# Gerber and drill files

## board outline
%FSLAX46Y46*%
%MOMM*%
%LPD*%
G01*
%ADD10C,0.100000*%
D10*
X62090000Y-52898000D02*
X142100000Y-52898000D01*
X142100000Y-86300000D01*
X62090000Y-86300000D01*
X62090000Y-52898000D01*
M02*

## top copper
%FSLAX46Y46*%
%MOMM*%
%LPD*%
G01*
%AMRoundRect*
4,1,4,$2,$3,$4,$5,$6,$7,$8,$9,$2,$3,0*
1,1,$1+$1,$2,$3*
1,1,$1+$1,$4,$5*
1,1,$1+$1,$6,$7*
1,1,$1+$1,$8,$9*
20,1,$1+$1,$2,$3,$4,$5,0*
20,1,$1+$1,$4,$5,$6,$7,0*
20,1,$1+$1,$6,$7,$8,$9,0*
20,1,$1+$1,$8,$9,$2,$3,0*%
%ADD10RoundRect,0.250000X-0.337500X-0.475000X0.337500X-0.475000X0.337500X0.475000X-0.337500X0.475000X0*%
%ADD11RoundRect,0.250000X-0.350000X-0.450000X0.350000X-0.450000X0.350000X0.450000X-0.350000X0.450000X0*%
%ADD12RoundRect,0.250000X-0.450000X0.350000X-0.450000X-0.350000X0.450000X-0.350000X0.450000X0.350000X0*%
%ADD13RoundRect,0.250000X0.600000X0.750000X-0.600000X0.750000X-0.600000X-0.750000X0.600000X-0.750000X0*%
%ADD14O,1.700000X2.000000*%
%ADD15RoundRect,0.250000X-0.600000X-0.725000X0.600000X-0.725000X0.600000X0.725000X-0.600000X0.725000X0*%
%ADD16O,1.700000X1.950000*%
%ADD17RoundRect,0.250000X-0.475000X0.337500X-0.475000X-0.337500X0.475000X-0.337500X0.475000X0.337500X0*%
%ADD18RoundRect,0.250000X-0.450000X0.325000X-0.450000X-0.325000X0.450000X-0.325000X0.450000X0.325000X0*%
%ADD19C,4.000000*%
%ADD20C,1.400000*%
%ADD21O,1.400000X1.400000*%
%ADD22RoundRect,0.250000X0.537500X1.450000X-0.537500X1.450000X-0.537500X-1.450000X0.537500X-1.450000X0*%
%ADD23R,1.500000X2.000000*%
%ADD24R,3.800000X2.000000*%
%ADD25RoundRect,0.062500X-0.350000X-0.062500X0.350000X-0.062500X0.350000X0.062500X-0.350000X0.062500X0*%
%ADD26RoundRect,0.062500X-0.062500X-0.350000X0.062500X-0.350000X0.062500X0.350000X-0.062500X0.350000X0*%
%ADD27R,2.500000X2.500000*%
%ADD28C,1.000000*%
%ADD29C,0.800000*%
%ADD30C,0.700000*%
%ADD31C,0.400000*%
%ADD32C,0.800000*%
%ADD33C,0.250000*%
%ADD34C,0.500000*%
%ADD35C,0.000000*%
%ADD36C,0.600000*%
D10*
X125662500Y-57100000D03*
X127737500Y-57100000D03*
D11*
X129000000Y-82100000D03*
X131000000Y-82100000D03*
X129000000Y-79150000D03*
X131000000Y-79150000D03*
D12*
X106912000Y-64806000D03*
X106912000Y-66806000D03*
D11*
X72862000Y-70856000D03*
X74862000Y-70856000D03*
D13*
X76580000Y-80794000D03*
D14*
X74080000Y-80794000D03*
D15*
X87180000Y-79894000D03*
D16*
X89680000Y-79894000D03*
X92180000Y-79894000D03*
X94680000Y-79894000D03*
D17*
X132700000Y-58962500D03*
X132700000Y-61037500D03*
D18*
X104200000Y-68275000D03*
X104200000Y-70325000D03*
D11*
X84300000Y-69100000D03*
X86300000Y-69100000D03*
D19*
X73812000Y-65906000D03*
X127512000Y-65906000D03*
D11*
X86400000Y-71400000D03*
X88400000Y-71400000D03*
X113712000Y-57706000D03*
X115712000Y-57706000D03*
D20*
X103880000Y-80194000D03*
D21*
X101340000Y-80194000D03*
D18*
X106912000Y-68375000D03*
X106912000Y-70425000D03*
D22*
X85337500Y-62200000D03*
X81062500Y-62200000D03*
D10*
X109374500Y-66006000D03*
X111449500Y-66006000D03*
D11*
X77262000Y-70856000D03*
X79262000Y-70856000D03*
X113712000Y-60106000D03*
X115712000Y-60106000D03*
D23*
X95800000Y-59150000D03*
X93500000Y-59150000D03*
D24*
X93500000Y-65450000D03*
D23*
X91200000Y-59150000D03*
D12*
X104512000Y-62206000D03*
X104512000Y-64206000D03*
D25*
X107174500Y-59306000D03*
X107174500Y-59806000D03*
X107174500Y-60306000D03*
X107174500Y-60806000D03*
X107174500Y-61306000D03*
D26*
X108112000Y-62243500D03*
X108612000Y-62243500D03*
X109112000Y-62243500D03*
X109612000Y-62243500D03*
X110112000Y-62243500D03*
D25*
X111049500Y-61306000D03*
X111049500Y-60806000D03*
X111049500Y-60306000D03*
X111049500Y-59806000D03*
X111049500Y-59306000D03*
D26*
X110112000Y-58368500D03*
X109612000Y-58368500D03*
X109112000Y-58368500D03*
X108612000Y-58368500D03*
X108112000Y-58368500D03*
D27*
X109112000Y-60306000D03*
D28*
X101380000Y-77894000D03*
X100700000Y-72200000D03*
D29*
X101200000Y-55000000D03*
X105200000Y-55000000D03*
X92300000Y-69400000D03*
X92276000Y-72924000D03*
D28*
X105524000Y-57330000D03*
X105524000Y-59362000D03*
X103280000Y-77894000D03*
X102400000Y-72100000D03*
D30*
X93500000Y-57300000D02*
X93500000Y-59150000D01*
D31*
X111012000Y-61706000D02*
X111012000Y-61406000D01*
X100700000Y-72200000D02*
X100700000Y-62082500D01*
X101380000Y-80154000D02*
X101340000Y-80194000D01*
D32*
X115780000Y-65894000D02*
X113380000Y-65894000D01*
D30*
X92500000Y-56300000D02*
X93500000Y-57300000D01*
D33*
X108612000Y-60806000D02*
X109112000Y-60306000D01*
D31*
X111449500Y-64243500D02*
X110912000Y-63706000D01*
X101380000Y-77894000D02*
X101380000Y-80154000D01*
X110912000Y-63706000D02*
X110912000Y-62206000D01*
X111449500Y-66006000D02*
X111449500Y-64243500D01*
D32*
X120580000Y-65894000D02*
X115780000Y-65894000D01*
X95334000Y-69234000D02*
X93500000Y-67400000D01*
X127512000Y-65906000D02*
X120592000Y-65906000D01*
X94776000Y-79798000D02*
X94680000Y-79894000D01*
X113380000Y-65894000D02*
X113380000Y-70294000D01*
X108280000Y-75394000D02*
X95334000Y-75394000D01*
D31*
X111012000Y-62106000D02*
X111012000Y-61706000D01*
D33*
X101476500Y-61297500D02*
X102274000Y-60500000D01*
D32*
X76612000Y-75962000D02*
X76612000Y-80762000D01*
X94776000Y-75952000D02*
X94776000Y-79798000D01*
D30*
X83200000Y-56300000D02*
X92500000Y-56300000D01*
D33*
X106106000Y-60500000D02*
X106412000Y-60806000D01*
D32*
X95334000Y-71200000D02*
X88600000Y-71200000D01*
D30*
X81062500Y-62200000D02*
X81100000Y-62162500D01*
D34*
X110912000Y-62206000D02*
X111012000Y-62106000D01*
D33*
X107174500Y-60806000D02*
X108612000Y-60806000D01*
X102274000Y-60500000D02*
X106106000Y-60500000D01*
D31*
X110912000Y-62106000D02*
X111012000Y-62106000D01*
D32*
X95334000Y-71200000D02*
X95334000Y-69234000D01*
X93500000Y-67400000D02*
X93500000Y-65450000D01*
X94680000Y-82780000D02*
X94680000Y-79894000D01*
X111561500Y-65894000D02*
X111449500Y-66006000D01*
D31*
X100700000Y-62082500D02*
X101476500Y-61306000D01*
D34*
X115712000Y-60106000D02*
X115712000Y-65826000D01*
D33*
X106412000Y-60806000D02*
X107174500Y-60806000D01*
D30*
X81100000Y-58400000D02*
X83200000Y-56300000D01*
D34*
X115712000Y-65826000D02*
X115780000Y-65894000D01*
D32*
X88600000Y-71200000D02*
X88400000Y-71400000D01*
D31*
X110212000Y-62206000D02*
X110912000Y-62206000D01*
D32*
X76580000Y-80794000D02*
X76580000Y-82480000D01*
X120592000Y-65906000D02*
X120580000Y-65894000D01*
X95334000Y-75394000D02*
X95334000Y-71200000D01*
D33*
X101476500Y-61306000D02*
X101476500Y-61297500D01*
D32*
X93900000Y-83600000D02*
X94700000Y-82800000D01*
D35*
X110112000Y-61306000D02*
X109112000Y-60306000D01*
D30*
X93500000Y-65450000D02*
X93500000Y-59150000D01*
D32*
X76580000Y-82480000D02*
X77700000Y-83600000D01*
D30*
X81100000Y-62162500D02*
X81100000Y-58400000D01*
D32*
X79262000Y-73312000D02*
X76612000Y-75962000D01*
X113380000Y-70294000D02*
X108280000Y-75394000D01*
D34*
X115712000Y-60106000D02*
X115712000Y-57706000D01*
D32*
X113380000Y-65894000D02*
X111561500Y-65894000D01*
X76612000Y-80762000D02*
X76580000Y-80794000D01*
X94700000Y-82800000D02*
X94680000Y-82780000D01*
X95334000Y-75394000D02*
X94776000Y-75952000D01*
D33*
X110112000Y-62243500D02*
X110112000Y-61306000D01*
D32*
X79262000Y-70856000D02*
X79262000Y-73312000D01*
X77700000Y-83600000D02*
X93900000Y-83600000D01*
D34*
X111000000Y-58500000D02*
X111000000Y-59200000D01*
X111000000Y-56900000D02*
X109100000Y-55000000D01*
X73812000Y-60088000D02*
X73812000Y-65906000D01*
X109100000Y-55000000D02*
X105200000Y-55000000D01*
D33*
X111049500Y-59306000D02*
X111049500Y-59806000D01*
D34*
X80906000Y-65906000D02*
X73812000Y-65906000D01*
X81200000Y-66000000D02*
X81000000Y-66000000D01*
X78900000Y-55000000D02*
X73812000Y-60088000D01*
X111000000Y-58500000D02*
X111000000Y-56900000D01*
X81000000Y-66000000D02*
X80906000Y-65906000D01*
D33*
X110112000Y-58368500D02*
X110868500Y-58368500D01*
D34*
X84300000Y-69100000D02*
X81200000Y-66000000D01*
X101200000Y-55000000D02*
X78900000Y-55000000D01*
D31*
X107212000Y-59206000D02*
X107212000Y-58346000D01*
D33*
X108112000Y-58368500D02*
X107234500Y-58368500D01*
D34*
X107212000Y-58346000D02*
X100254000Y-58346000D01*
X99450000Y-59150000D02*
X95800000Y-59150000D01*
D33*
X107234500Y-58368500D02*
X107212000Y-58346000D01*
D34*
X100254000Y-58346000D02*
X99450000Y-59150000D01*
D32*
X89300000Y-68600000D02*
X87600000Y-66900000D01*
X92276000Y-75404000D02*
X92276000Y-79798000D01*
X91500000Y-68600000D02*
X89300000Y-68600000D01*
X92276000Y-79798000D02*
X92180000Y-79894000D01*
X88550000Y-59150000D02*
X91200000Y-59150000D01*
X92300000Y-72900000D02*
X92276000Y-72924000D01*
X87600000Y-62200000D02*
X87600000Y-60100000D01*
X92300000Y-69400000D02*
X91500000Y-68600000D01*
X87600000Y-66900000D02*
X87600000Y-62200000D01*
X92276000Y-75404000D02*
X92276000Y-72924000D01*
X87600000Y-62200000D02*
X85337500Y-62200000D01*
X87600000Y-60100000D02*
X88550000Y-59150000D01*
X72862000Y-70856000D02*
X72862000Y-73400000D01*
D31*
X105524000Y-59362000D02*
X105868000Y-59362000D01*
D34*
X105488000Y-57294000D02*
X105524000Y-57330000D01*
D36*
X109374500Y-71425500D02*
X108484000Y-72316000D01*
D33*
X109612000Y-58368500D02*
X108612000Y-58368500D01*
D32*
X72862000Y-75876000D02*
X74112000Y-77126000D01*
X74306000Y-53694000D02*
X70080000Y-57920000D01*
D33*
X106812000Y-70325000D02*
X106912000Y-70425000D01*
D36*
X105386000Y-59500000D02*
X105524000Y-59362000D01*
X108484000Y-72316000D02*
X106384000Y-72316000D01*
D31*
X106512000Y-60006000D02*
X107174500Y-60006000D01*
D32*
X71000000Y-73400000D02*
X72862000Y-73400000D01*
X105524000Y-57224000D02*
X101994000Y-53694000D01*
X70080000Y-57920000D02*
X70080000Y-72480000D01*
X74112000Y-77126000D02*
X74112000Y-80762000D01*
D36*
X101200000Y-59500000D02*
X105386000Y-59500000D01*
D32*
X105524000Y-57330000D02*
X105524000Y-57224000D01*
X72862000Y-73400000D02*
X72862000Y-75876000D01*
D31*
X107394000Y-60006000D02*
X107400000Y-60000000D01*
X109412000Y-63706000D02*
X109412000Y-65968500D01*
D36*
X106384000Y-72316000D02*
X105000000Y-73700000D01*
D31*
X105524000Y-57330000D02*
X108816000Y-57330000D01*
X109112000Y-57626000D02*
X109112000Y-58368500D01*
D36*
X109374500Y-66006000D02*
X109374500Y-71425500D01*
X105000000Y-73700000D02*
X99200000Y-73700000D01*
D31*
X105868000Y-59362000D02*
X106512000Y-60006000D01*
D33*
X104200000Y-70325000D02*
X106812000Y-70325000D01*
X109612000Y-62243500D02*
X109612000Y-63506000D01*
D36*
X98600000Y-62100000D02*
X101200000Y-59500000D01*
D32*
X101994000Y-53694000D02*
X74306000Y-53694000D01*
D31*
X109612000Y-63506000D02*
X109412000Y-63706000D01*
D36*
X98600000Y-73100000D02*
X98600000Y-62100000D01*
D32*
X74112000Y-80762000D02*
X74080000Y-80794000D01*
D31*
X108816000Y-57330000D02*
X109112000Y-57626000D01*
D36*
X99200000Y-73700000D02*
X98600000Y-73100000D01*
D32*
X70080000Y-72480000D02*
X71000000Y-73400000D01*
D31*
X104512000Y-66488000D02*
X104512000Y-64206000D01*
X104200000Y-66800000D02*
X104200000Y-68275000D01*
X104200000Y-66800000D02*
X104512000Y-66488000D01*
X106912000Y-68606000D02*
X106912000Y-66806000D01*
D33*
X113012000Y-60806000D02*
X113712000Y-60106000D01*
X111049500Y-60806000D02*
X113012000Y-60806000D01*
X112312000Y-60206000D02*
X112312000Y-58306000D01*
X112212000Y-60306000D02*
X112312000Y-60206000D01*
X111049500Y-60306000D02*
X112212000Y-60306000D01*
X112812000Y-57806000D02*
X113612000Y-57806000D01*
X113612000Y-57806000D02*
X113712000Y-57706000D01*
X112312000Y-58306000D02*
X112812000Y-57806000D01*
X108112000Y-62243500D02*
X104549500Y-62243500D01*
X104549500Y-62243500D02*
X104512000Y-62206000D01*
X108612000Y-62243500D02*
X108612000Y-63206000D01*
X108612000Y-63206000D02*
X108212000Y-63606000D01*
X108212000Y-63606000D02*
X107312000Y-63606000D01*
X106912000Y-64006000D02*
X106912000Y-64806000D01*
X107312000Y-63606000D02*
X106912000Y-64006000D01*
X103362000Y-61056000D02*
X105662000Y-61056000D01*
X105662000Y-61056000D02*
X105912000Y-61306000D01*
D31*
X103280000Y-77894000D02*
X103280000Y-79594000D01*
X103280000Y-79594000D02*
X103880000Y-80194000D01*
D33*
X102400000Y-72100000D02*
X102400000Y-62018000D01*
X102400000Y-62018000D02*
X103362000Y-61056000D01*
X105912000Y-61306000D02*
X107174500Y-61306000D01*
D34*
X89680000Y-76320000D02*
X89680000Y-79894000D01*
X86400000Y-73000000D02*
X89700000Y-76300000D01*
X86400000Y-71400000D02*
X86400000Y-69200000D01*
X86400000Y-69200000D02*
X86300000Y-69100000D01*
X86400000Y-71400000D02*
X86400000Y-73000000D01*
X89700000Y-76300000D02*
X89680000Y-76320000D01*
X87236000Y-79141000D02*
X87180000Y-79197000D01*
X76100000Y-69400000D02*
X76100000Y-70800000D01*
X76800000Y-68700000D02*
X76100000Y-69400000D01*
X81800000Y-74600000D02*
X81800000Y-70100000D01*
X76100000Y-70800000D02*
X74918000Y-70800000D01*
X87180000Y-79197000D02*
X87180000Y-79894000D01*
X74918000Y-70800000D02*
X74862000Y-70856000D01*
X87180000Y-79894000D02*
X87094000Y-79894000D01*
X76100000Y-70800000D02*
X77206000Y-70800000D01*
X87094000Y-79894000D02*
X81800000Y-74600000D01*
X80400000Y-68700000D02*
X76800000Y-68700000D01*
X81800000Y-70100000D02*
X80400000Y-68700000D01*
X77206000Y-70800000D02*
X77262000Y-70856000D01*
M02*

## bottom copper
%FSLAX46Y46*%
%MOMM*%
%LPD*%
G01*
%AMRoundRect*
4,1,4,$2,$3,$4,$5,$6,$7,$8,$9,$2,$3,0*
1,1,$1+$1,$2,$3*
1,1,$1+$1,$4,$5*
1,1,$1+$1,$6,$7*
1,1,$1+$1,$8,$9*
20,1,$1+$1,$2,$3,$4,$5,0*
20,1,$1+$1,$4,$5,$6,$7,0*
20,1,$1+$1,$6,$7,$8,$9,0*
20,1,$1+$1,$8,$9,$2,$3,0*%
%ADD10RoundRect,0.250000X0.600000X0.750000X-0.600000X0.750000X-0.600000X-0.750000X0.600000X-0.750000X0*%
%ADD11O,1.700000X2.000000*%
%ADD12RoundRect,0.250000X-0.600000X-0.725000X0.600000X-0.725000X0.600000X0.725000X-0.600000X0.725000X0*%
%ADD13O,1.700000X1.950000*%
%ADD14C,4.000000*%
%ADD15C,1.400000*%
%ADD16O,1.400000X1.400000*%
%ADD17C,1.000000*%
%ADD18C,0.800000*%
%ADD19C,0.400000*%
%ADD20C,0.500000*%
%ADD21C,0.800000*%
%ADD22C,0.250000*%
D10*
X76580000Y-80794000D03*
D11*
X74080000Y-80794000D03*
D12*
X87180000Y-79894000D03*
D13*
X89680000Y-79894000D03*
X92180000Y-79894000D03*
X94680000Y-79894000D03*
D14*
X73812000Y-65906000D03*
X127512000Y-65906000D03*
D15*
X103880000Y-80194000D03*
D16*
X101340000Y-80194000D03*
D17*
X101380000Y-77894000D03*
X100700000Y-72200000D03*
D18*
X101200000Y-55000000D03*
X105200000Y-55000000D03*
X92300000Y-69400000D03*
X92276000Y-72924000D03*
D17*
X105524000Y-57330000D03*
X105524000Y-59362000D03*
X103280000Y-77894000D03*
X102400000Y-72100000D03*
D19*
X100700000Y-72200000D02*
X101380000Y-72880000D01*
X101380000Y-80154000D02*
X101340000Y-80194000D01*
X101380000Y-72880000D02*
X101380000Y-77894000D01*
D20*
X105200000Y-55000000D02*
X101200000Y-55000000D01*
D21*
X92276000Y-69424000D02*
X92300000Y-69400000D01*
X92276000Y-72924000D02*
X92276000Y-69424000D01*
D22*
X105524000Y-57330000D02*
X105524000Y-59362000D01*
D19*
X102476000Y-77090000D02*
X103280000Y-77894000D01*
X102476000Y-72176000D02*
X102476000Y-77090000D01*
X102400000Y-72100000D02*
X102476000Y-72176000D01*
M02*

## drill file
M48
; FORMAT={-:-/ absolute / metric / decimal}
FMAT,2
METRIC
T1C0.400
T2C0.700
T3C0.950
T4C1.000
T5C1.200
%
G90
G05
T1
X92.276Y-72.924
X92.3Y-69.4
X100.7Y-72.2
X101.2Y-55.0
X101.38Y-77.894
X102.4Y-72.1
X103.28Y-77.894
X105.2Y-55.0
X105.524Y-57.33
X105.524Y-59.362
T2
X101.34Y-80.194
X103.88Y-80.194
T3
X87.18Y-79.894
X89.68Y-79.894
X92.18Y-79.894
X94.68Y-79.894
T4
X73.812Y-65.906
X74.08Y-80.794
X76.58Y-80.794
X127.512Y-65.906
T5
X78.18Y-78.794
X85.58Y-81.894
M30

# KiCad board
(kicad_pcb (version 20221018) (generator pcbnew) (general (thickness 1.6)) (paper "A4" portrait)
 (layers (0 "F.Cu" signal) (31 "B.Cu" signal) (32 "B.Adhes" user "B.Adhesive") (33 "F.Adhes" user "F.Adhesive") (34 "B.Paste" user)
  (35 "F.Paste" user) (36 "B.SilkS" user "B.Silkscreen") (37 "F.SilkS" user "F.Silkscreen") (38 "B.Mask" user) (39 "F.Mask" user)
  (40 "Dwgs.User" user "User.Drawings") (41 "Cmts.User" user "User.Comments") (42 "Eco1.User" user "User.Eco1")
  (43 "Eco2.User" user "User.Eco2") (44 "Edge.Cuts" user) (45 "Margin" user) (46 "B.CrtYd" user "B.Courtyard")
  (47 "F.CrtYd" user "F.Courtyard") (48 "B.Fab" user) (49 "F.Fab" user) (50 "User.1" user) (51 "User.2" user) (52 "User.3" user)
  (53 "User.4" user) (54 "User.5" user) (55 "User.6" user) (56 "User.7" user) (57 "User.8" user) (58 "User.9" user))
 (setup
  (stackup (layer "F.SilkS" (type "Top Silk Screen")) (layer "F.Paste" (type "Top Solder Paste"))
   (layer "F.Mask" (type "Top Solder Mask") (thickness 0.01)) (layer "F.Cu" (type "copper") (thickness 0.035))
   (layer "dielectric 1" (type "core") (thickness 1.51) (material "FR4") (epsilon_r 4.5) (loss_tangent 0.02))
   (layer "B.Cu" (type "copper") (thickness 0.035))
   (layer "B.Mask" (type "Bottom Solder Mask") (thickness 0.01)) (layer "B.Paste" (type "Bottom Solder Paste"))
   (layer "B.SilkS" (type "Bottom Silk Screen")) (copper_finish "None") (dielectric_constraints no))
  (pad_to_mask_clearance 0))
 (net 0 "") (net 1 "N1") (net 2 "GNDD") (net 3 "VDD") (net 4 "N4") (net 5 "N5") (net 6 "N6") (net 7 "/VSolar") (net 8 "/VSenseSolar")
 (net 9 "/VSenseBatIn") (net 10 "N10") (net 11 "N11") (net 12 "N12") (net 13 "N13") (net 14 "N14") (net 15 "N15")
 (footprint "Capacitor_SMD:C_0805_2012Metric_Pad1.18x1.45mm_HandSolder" (layer "F.Cu") (at 126.7 57.1)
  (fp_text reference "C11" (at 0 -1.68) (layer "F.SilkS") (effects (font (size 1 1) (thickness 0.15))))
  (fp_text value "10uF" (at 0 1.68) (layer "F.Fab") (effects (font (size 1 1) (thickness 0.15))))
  (pad "1" smd roundrect (at -1.0375 0) (size 1.175 1.45) (layers "F.Cu" "F.Paste" "F.Mask") (roundrect_rratio 0.212766) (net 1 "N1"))
  (pad "2" smd roundrect (at 1.0375 0) (size 1.175 1.45) (layers "F.Cu" "F.Paste" "F.Mask") (roundrect_rratio 0.212766) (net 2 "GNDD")))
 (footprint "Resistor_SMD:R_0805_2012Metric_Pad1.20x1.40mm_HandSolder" (layer "F.Cu") (at 130 82.1)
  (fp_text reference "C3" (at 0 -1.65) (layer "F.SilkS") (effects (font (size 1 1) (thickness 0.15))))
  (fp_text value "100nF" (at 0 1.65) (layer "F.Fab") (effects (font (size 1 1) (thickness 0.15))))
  (pad "1" smd roundrect (at -1 0) (size 1.2 1.4) (layers "F.Cu" "F.Paste" "F.Mask") (roundrect_rratio 0.208333) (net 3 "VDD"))
  (pad "2" smd roundrect (at 1 0) (size 1.2 1.4) (layers "F.Cu" "F.Paste" "F.Mask") (roundrect_rratio 0.208333) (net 2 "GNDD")))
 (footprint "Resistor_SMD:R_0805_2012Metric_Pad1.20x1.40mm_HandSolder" (layer "F.Cu") (at 130 79.15)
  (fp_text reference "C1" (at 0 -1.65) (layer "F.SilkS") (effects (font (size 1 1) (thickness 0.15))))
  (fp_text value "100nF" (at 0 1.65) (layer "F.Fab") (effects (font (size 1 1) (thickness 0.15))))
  (pad "1" smd roundrect (at -1 0) (size 1.2 1.4) (layers "F.Cu" "F.Paste" "F.Mask") (roundrect_rratio 0.208333) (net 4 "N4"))
  (pad "2" smd roundrect (at 1 0) (size 1.2 1.4) (layers "F.Cu" "F.Paste" "F.Mask") (roundrect_rratio 0.208333) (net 2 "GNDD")))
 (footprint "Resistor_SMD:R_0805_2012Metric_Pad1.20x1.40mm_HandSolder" (layer "F.Cu") (at 106.912 65.806 -90)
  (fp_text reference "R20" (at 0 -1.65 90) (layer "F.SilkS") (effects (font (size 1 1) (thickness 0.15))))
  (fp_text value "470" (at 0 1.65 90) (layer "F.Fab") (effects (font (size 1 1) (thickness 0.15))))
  (pad "1" smd roundrect (at -1 0 270) (size 1.2 1.4) (layers "F.Cu" "F.Paste" "F.Mask") (roundrect_rratio 0.208333) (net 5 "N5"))
  (pad "2" smd roundrect (at 1 0 270) (size 1.2 1.4) (layers "F.Cu" "F.Paste" "F.Mask") (roundrect_rratio 0.208333) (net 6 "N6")))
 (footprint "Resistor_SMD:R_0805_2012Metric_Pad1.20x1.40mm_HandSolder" (layer "F.Cu") (at 73.862 70.856)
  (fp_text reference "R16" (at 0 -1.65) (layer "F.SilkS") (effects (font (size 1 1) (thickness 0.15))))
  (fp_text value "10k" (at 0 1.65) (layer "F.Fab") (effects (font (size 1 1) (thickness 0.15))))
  (pad "1" smd roundrect (at -1 0) (size 1.2 1.4) (layers "F.Cu" "F.Paste" "F.Mask") (roundrect_rratio 0.208333) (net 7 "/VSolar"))
  (pad "2" smd roundrect (at 1 0) (size 1.2 1.4) (layers "F.Cu" "F.Paste" "F.Mask") (roundrect_rratio 0.208333) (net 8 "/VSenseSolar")))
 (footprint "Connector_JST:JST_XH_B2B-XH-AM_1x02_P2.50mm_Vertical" (layer "F.Cu") (at 76.58 80.794 180)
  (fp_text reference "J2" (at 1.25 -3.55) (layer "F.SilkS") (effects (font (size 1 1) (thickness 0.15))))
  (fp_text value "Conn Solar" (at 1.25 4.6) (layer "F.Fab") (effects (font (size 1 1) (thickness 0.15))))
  (pad "" np_thru_hole circle (at -1.6 2 180) (size 1.2 1.2) (drill 1.2) (layers "*.Cu" "*.Mask"))
  (pad "1" thru_hole roundrect (at 0 0 180) (size 1.7 2) (drill 1) (layers "*.Cu" "*.Mask") (roundrect_rratio 0.147059) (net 2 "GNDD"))
  (pad "2" thru_hole oval (at 2.5 0 180) (size 1.7 2) (drill 1) (layers "*.Cu" "*.Mask") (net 7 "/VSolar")))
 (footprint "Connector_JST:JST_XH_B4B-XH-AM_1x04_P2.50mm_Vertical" (layer "F.Cu") (at 87.18 79.894)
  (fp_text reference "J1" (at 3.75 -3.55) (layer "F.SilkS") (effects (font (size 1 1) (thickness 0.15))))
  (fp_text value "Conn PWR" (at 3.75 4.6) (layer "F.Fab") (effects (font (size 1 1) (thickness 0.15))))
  (pad "" np_thru_hole circle (at -1.6 2) (size 1.2 1.2) (drill 1.2) (layers "*.Cu" "*.Mask"))
  (pad "1" thru_hole roundrect (at 0 0) (size 1.7 1.95) (drill 0.95) (layers "*.Cu" "*.Mask") (roundrect_rratio 0.147059)
   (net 8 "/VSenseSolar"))
  (pad "2" thru_hole oval (at 2.5 0) (size 1.7 1.95) (drill 0.95) (layers "*.Cu" "*.Mask") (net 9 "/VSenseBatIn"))
  (pad "3" thru_hole oval (at 5 0) (size 1.7 1.95) (drill 0.95) (layers "*.Cu" "*.Mask") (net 3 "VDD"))
  (pad "4" thru_hole oval (at 7.5 0) (size 1.7 1.95) (drill 0.95) (layers "*.Cu" "*.Mask") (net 2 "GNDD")))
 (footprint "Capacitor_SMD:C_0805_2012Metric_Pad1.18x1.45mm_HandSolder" (layer "F.Cu") (at 132.7 60 -90)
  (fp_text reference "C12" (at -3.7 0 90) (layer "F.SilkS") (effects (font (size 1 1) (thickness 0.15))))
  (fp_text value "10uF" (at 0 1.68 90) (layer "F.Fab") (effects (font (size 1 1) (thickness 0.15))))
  (pad "1" smd roundrect (at -1.0375 0 270) (size 1.175 1.45) (layers "F.Cu" "F.Paste" "F.Mask") (roundrect_rratio 0.212766) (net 4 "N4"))
  (pad "2" smd roundrect (at 1.0375 0 270) (size 1.175 1.45) (layers "F.Cu" "F.Paste" "F.Mask") (roundrect_rratio 0.212766) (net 2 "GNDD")))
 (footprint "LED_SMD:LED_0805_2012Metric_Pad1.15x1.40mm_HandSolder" (layer "F.Cu") (at 104.2 69.3 -90)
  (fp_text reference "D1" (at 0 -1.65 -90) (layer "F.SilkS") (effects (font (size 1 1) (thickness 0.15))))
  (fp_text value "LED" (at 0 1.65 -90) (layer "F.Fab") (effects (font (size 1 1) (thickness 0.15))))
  (pad "1" smd roundrect (at -1.025 0 270) (size 1.15 1.4) (layers "F.Cu" "F.Paste" "F.Mask") (roundrect_rratio 0.217391) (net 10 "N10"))
  (pad "2" smd roundrect (at 1.025 0 270) (size 1.15 1.4) (layers "F.Cu" "F.Paste" "F.Mask") (roundrect_rratio 0.217391) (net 7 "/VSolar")))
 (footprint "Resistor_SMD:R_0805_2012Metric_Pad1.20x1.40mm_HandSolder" (layer "F.Cu") (at 85.3 69.1)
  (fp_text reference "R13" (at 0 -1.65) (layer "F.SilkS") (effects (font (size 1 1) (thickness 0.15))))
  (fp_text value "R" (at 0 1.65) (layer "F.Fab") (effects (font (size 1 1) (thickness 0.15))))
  (pad "1" smd roundrect (at -1 0) (size 1.2 1.4) (layers "F.Cu" "F.Paste" "F.Mask") (roundrect_rratio 0.208333) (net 1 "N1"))
  (pad "2" smd roundrect (at 1 0) (size 1.2 1.4) (layers "F.Cu" "F.Paste" "F.Mask") (roundrect_rratio 0.208333) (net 9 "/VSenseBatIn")))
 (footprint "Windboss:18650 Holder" (layer "F.Cu") (at 74.512 65.906)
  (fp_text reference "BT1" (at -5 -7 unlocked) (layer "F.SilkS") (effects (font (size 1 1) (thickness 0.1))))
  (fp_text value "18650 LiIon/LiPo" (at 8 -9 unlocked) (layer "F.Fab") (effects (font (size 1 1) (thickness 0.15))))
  (pad "1" thru_hole circle (at -0.7 0) (size 4 4) (drill 1) (layers "*.Cu" "*.Mask") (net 1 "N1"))
  (pad "2" thru_hole circle (at 53 0) (size 4 4) (drill 1) (layers "*.Cu" "*.Mask") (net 2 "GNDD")))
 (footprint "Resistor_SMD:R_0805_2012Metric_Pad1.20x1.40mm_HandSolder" (layer "F.Cu") (at 87.4 71.4)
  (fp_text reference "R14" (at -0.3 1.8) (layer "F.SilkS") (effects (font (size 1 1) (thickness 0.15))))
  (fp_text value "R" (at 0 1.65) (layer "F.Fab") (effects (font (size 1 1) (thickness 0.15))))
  (pad "1" smd roundrect (at -1 0) (size 1.2 1.4) (layers "F.Cu" "F.Paste" "F.Mask") (roundrect_rratio 0.208333) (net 9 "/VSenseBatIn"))
  (pad "2" smd roundrect (at 1 0) (size 1.2 1.4) (layers "F.Cu" "F.Paste" "F.Mask") (roundrect_rratio 0.208333) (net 2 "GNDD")))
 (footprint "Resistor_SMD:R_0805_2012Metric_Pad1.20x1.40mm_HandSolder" (layer "F.Cu") (at 114.712 57.706)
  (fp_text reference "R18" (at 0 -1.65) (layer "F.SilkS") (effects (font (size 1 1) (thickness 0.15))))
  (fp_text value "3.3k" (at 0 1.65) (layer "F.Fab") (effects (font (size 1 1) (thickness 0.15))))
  (pad "1" smd roundrect (at -1 0) (size 1.2 1.4) (layers "F.Cu" "F.Paste" "F.Mask") (roundrect_rratio 0.208333) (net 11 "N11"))
  (pad "2" smd roundrect (at 1 0) (size 1.2 1.4) (layers "F.Cu" "F.Paste" "F.Mask") (roundrect_rratio 0.208333) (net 2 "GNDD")))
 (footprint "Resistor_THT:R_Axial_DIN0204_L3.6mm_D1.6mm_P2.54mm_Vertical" (layer "F.Cu") (at 103.88 80.194 180)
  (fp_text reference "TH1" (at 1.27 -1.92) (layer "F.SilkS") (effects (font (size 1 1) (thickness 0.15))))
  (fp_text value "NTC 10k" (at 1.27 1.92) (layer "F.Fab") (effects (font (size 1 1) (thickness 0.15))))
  (pad "1" thru_hole circle (at 0 0 180) (size 1.4 1.4) (drill 0.7) (layers "*.Cu" "*.Mask") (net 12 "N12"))
  (pad "2" thru_hole oval (at 2.54 0 180) (size 1.4 1.4) (drill 0.7) (layers "*.Cu" "*.Mask") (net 2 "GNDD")))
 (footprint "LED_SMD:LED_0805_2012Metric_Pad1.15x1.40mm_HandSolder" (layer "F.Cu") (at 106.912 69.4 -90)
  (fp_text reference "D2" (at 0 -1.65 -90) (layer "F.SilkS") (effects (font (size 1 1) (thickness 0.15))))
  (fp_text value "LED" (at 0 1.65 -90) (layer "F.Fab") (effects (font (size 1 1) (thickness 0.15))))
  (pad "1" smd roundrect (at -1.025 0 270) (size 1.15 1.4) (layers "F.Cu" "F.Paste" "F.Mask") (roundrect_rratio 0.217391) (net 6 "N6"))
  (pad "2" smd roundrect (at 1.025 0 270) (size 1.15 1.4) (layers "F.Cu" "F.Paste" "F.Mask") (roundrect_rratio 0.217391) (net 7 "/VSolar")))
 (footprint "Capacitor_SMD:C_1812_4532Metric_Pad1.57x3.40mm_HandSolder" (layer "F.Cu") (at 83.2 62.2 180)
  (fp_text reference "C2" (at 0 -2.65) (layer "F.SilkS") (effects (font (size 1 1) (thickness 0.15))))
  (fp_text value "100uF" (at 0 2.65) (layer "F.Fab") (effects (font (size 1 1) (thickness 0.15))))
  (pad "1" smd roundrect (at -2.1375 0 180) (size 1.575 3.4) (layers "F.Cu" "F.Paste" "F.Mask") (roundrect_rratio 0.15873) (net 3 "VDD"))
  (pad "2" smd roundrect (at 2.1375 0 180) (size 1.575 3.4) (layers "F.Cu" "F.Paste" "F.Mask") (roundrect_rratio 0.15873) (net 2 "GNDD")))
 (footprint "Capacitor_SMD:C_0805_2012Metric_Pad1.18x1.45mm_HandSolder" (layer "F.Cu") (at 110.412 66.006)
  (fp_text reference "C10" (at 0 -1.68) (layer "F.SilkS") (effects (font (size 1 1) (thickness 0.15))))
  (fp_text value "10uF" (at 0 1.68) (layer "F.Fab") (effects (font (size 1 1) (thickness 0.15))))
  (pad "1" smd roundrect (at -1.0375 0) (size 1.175 1.45) (layers "F.Cu" "F.Paste" "F.Mask") (roundrect_rratio 0.212766) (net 7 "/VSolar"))
  (pad "2" smd roundrect (at 1.0375 0) (size 1.175 1.45) (layers "F.Cu" "F.Paste" "F.Mask") (roundrect_rratio 0.212766) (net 2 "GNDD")))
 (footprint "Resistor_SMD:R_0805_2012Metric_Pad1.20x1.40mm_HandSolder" (layer "F.Cu") (at 78.262 70.856)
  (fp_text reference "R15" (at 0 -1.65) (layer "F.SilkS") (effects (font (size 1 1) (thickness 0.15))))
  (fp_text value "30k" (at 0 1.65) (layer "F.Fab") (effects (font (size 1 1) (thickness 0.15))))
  (pad "1" smd roundrect (at -1 0) (size 1.2 1.4) (layers "F.Cu" "F.Paste" "F.Mask") (roundrect_rratio 0.208333) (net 8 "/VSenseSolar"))
  (pad "2" smd roundrect (at 1 0) (size 1.2 1.4) (layers "F.Cu" "F.Paste" "F.Mask") (roundrect_rratio 0.208333) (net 2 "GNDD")))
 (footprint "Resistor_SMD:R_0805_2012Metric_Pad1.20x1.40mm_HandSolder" (layer "F.Cu") (at 114.712 60.106)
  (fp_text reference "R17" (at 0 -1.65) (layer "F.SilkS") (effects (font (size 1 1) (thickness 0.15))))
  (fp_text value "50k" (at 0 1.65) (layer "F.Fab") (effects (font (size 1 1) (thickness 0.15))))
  (pad "1" smd roundrect (at -1 0) (size 1.2 1.4) (layers "F.Cu" "F.Paste" "F.Mask") (roundrect_rratio 0.208333) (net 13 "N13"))
  (pad "2" smd roundrect (at 1 0) (size 1.2 1.4) (layers "F.Cu" "F.Paste" "F.Mask") (roundrect_rratio 0.208333) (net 2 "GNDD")))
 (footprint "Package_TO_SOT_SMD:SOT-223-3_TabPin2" (layer "F.Cu") (at 93.5 62.3 -90)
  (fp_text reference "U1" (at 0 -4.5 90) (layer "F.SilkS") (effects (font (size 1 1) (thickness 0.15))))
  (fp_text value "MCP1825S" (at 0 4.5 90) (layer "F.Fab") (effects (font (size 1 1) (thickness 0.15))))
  (pad "1" smd rect (at -3.15 -2.3 270) (size 2 1.5) (layers "F.Cu" "F.Paste" "F.Mask") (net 4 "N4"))
  (pad "2" smd rect (at -3.15 0 270) (size 2 1.5) (layers "F.Cu" "F.Paste" "F.Mask") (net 2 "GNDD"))
  (pad "2" smd rect (at 3.15 0 270) (size 2 3.8) (layers "F.Cu" "F.Paste" "F.Mask") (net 2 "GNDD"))
  (pad "3" smd rect (at -3.15 2.3 270) (size 2 1.5) (layers "F.Cu" "F.Paste" "F.Mask") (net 3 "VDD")))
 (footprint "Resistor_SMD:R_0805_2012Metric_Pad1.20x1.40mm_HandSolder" (layer "F.Cu") (at 104.512 63.206 -90)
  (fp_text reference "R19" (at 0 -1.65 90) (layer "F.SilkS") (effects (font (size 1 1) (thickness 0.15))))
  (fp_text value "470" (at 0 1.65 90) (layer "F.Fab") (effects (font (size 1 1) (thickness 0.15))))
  (pad "1" smd roundrect (at -1 0 270) (size 1.2 1.4) (layers "F.Cu" "F.Paste" "F.Mask") (roundrect_rratio 0.208333) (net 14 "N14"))
  (pad "2" smd roundrect (at 1 0 270) (size 1.2 1.4) (layers "F.Cu" "F.Paste" "F.Mask") (roundrect_rratio 0.208333) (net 10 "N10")))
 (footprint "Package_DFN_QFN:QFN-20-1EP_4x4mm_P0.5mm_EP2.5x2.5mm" (layer "F.Cu") (at 109.112 60.306)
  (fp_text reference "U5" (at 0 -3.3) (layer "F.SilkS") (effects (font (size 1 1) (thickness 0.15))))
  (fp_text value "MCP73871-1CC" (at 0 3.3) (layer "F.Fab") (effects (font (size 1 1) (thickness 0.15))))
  (pad "" smd roundrect (at -0.625 -0.625) (size 1.01 1.01) (layers "F.Paste") (roundrect_rratio 0.247525))
  (pad "" smd roundrect (at -0.625 0.625) (size 1.01 1.01) (layers "F.Paste") (roundrect_rratio 0.247525))
  (pad "" smd roundrect (at 0.625 -0.625) (size 1.01 1.01) (layers "F.Paste") (roundrect_rratio 0.247525))
  (pad "" smd roundrect (at 0.625 0.625) (size 1.01 1.01) (layers "F.Paste") (roundrect_rratio 0.247525))
  (pad "1" smd roundrect (at -1.9375 -1) (size 0.825 0.25) (layers "F.Cu" "F.Paste" "F.Mask") (roundrect_rratio 0.25) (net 4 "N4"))
  (pad "2" smd roundrect (at -1.9375 -0.5) (size 0.825 0.25) (layers "F.Cu" "F.Paste" "F.Mask") (roundrect_rratio 0.25) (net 7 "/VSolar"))
  (pad "3" smd roundrect (at -1.9375 0) (size 0.825 0.25) (layers "F.Cu" "F.Paste" "F.Mask") (roundrect_rratio 0.25) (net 7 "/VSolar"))
  (pad "4" smd roundrect (at -1.9375 0.5) (size 0.825 0.25) (layers "F.Cu" "F.Paste" "F.Mask") (roundrect_rratio 0.25) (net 2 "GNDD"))
  (pad "5" smd roundrect (at -1.9375 1) (size 0.825 0.25) (layers "F.Cu" "F.Paste" "F.Mask") (roundrect_rratio 0.25) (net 12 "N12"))
  (pad "6" smd roundrect (at -1 1.9375) (size 0.25 0.825) (layers "F.Cu" "F.Paste" "F.Mask") (roundrect_rratio 0.25) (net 14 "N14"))
  (pad "7" smd roundrect (at -0.5 1.9375) (size 0.25 0.825) (layers "F.Cu" "F.Paste" "F.Mask") (roundrect_rratio 0.25) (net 5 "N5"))
  (pad "8" smd roundrect (at 0 1.9375) (size 0.25 0.825) (layers "F.Cu" "F.Paste" "F.Mask") (roundrect_rratio 0.25) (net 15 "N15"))
  (pad "9" smd roundrect (at 0.5 1.9375) (size 0.25 0.825) (layers "F.Cu" "F.Paste" "F.Mask") (roundrect_rratio 0.25) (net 7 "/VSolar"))
  (pad "10" smd roundrect (at 1 1.9375) (size 0.25 0.825) (layers "F.Cu" "F.Paste" "F.Mask") (roundrect_rratio 0.25) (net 2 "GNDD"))
  (pad "11" smd roundrect (at 1.9375 1) (size 0.825 0.25) (layers "F.Cu" "F.Paste" "F.Mask") (roundrect_rratio 0.25) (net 2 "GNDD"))
  (pad "12" smd roundrect (at 1.9375 0.5) (size 0.825 0.25) (layers "F.Cu" "F.Paste" "F.Mask") (roundrect_rratio 0.25) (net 13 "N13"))
  (pad "13" smd roundrect (at 1.9375 0) (size 0.825 0.25) (layers "F.Cu" "F.Paste" "F.Mask") (roundrect_rratio 0.25) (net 11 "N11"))
  (pad "14" smd roundrect (at 1.9375 -0.5) (size 0.825 0.25) (layers "F.Cu" "F.Paste" "F.Mask") (roundrect_rratio 0.25) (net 1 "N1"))
  (pad "15" smd roundrect (at 1.9375 -1) (size 0.825 0.25) (layers "F.Cu" "F.Paste" "F.Mask") (roundrect_rratio 0.25) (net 1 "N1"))
  (pad "16" smd roundrect (at 1 -1.9375) (size 0.25 0.825) (layers "F.Cu" "F.Paste" "F.Mask") (roundrect_rratio 0.25) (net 1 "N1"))
  (pad "17" smd roundrect (at 0.5 -1.9375) (size 0.25 0.825) (layers "F.Cu" "F.Paste" "F.Mask") (roundrect_rratio 0.25) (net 7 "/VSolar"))
  (pad "18" smd roundrect (at 0 -1.9375) (size 0.25 0.825) (layers "F.Cu" "F.Paste" "F.Mask") (roundrect_rratio 0.25) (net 7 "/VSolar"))
  (pad "19" smd roundrect (at -0.5 -1.9375) (size 0.25 0.825) (layers "F.Cu" "F.Paste" "F.Mask") (roundrect_rratio 0.25) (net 7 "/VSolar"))
  (pad "20" smd roundrect (at -1 -1.9375) (size 0.25 0.825) (layers "F.Cu" "F.Paste" "F.Mask") (roundrect_rratio 0.25) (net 4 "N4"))
  (pad "21" smd rect (at 0 0) (size 2.5 2.5) (layers "F.Cu" "F.Mask") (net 2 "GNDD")))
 (gr_rect (start 62.09 52.898) (end 142.1 86.3) (stroke (width 0.1) (type default)) (fill none) (layer "Edge.Cuts"))
 (segment (start 93.5 57.3) (end 93.5 59.15) (width 0.7) (layer "F.Cu") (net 2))
 (segment (start 111.012 61.706) (end 111.012 61.406) (width 0.4) (layer "F.Cu") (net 2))
 (segment (start 100.7 72.2) (end 100.7 62.0825) (width 0.4) (layer "F.Cu") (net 2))
 (segment (start 101.38 80.154) (end 101.34 80.194) (width 0.4) (layer "F.Cu") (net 2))
 (segment (start 115.78 65.894) (end 113.38 65.894) (width 0.8) (layer "F.Cu") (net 2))
 (segment (start 92.5 56.3) (end 93.5 57.3) (width 0.7) (layer "F.Cu") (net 2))
 (segment (start 108.612 60.806) (end 109.112 60.306) (width 0.25) (layer "F.Cu") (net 2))
 (segment (start 111.4495 64.2435) (end 110.912 63.706) (width 0.4) (layer "F.Cu") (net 2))
 (segment (start 101.38 77.894) (end 101.38 80.154) (width 0.4) (layer "F.Cu") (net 2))
 (segment (start 110.912 63.706) (end 110.912 62.206) (width 0.4) (layer "F.Cu") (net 2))
 (segment (start 111.4495 66.006) (end 111.4495 64.2435) (width 0.4) (layer "F.Cu") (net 2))
 (segment (start 120.58 65.894) (end 115.78 65.894) (width 0.8) (layer "F.Cu") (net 2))
 (segment (start 95.334 69.234) (end 93.5 67.4) (width 0.8) (layer "F.Cu") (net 2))
 (segment (start 127.512 65.906) (end 120.592 65.906) (width 0.8) (layer "F.Cu") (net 2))
 (segment (start 94.776 79.798) (end 94.68 79.894) (width 0.8) (layer "F.Cu") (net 2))
 (segment (start 113.38 65.894) (end 113.38 70.294) (width 0.8) (layer "F.Cu") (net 2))
 (segment (start 108.28 75.394) (end 95.334 75.394) (width 0.8) (layer "F.Cu") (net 2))
 (segment (start 111.012 62.106) (end 111.012 61.706) (width 0.4) (layer "F.Cu") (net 2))
 (segment (start 101.4765 61.2975) (end 102.274 60.5) (width 0.25) (layer "F.Cu") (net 2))
 (segment (start 76.612 75.962) (end 76.612 80.762) (width 0.8) (layer "F.Cu") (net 2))
 (segment (start 94.776 75.952) (end 94.776 79.798) (width 0.8) (layer "F.Cu") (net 2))
 (segment (start 83.2 56.3) (end 92.5 56.3) (width 0.7) (layer "F.Cu") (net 2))
 (segment (start 106.106 60.5) (end 106.412 60.806) (width 0.25) (layer "F.Cu") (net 2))
 (segment (start 95.334 71.2) (end 88.6 71.2) (width 0.8) (layer "F.Cu") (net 2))
 (segment (start 81.0625 62.2) (end 81.1 62.1625) (width 0.7) (layer "F.Cu") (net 2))
 (segment (start 110.912 62.206) (end 111.012 62.106) (width 0.5) (layer "F.Cu") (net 2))
 (segment (start 107.1745 60.806) (end 108.612 60.806) (width 0.25) (layer "F.Cu") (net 2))
 (segment (start 102.274 60.5) (end 106.106 60.5) (width 0.25) (layer "F.Cu") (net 2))
 (segment (start 110.912 62.106) (end 111.012 62.106) (width 0.4) (layer "F.Cu") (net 2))
 (segment (start 95.334 71.2) (end 95.334 69.234) (width 0.8) (layer "F.Cu") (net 2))
 (segment (start 93.5 67.4) (end 93.5 65.45) (width 0.8) (layer "F.Cu") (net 2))
 (segment (start 94.68 82.78) (end 94.68 79.894) (width 0.8) (layer "F.Cu") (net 2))
 (segment (start 111.5615 65.894) (end 111.4495 66.006) (width 0.8) (layer "F.Cu") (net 2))
 (segment (start 100.7 62.0825) (end 101.4765 61.306) (width 0.4) (layer "F.Cu") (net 2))
 (segment (start 115.712 60.106) (end 115.712 65.826) (width 0.5) (layer "F.Cu") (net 2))
 (segment (start 106.412 60.806) (end 107.1745 60.806) (width 0.25) (layer "F.Cu") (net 2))
 (segment (start 81.1 58.4) (end 83.2 56.3) (width 0.7) (layer "F.Cu") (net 2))
 (segment (start 115.712 65.826) (end 115.78 65.894) (width 0.5) (layer "F.Cu") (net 2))
 (segment (start 88.6 71.2) (end 88.4 71.4) (width 0.8) (layer "F.Cu") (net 2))
 (segment (start 110.212 62.206) (end 110.912 62.206) (width 0.4) (layer "F.Cu") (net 2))
 (segment (start 76.58 80.794) (end 76.58 82.48) (width 0.8) (layer "F.Cu") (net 2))
 (segment (start 120.592 65.906) (end 120.58 65.894) (width 0.8) (layer "F.Cu") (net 2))
 (segment (start 95.334 75.394) (end 95.334 71.2) (width 0.8) (layer "F.Cu") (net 2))
 (segment (start 101.4765 61.306) (end 101.4765 61.2975) (width 0.25) (layer "F.Cu") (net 2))
 (segment (start 93.9 83.6) (end 94.7 82.8) (width 0.8) (layer "F.Cu") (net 2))
 (segment (start 110.112 61.306) (end 109.112 60.306) (width 0) (layer "F.Cu") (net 2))
 (segment (start 93.5 65.45) (end 93.5 59.15) (width 0.7) (layer "F.Cu") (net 2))
 (segment (start 76.58 82.48) (end 77.7 83.6) (width 0.8) (layer "F.Cu") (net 2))
 (segment (start 81.1 62.1625) (end 81.1 58.4) (width 0.7) (layer "F.Cu") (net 2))
 (segment (start 79.262 73.312) (end 76.612 75.962) (width 0.8) (layer "F.Cu") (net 2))
 (segment (start 113.38 70.294) (end 108.28 75.394) (width 0.8) (layer "F.Cu") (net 2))
 (segment (start 115.712 60.106) (end 115.712 57.706) (width 0.5) (layer "F.Cu") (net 2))
 (segment (start 113.38 65.894) (end 111.5615 65.894) (width 0.8) (layer "F.Cu") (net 2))
 (segment (start 76.612 80.762) (end 76.58 80.794) (width 0.8) (layer "F.Cu") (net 2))
 (segment (start 94.7 82.8) (end 94.68 82.78) (width 0.8) (layer "F.Cu") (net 2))
 (segment (start 95.334 75.394) (end 94.776 75.952) (width 0.8) (layer "F.Cu") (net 2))
 (segment (start 110.112 62.2435) (end 110.112 61.306) (width 0.25) (layer "F.Cu") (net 2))
 (segment (start 79.262 70.856) (end 79.262 73.312) (width 0.8) (layer "F.Cu") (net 2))
 (segment (start 77.7 83.6) (end 93.9 83.6) (width 0.8) (layer "F.Cu") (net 2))
 (via (at 101.38 77.894) (size 1) (drill 0.4) (layers "F.Cu" "B.Cu") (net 2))
 (via (at 100.7 72.2) (size 1) (drill 0.4) (layers "F.Cu" "B.Cu") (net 2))
 (segment (start 100.7 72.2) (end 101.38 72.88) (width 0.4) (layer "B.Cu") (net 2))
 (segment (start 101.38 80.154) (end 101.34 80.194) (width 0.4) (layer "B.Cu") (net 2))
 (segment (start 101.38 72.88) (end 101.38 77.894) (width 0.4) (layer "B.Cu") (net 2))
 (segment (start 111 58.5) (end 111 59.2) (width 0.5) (layer "F.Cu") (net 1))
 (segment (start 111 56.9) (end 109.1 55) (width 0.5) (layer "F.Cu") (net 1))
 (segment (start 73.812 60.088) (end 73.812 65.906) (width 0.5) (layer "F.Cu") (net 1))
 (segment (start 109.1 55) (end 105.2 55) (width 0.5) (layer "F.Cu") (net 1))
 (segment (start 111.0495 59.306) (end 111.0495 59.806) (width 0.25) (layer "F.Cu") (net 1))
 (segment (start 80.906 65.906) (end 73.812 65.906) (width 0.5) (layer "F.Cu") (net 1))
 (segment (start 81.2 66) (end 81 66) (width 0.5) (layer "F.Cu") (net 1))
 (segment (start 78.9 55) (end 73.812 60.088) (width 0.5) (layer "F.Cu") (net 1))
 (segment (start 111 58.5) (end 111 56.9) (width 0.5) (layer "F.Cu") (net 1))
 (segment (start 81 66) (end 80.906 65.906) (width 0.5) (layer "F.Cu") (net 1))
 (segment (start 110.112 58.3685) (end 110.8685 58.3685) (width 0.25) (layer "F.Cu") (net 1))
 (segment (start 84.3 69.1) (end 81.2 66) (width 0.5) (layer "F.Cu") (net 1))
 (segment (start 101.2 55) (end 78.9 55) (width 0.5) (layer "F.Cu") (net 1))
 (via (at 101.2 55) (size 0.8) (drill 0.4) (layers "F.Cu" "B.Cu") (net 1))
 (via (at 105.2 55) (size 0.8) (drill 0.4) (layers "F.Cu" "B.Cu") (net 1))
 (segment (start 105.2 55) (end 101.2 55) (width 0.5) (layer "B.Cu") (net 1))
 (segment (start 107.212 59.206) (end 107.212 58.346) (width 0.4) (layer "F.Cu") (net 4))
 (segment (start 108.112 58.3685) (end 107.2345 58.3685) (width 0.25) (layer "F.Cu") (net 4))
 (segment (start 107.212 58.346) (end 100.254 58.346) (width 0.5) (layer "F.Cu") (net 4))
 (segment (start 99.45 59.15) (end 95.8 59.15) (width 0.5) (layer "F.Cu") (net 4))
 (segment (start 107.2345 58.3685) (end 107.212 58.346) (width 0.25) (layer "F.Cu") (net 4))
 (segment (start 100.254 58.346) (end 99.45 59.15) (width 0.5) (layer "F.Cu") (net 4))
 (segment (start 89.3 68.6) (end 87.6 66.9) (width 0.8) (layer "F.Cu") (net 3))
 (segment (start 92.276 75.404) (end 92.276 79.798) (width 0.8) (layer "F.Cu") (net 3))
 (segment (start 91.5 68.6) (end 89.3 68.6) (width 0.8) (layer "F.Cu") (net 3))
 (segment (start 92.276 79.798) (end 92.18 79.894) (width 0.8) (layer "F.Cu") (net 3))
 (segment (start 88.55 59.15) (end 91.2 59.15) (width 0.8) (layer "F.Cu") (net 3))
 (segment (start 92.3 72.9) (end 92.276 72.924) (width 0.8) (layer "F.Cu") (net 3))
 (segment (start 87.6 62.2) (end 87.6 60.1) (width 0.8) (layer "F.Cu") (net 3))
 (segment (start 92.3 69.4) (end 91.5 68.6) (width 0.8) (layer "F.Cu") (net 3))
 (segment (start 87.6 66.9) (end 87.6 62.2) (width 0.8) (layer "F.Cu") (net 3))
 (segment (start 92.276 75.404) (end 92.276 72.924) (width 0.8) (layer "F.Cu") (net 3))
 (segment (start 87.6 62.2) (end 85.3375 62.2) (width 0.8) (layer "F.Cu") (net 3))
 (segment (start 87.6 60.1) (end 88.55 59.15) (width 0.8) (layer "F.Cu") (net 3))
 (via (at 92.3 69.4) (size 0.8) (drill 0.4) (layers "F.Cu" "B.Cu") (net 3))
 (via (at 92.276 72.924) (size 0.8) (drill 0.4) (layers "F.Cu" "B.Cu") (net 3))
 (segment (start 92.276 69.424) (end 92.3 69.4) (width 0.8) (layer "B.Cu") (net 3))
 (segment (start 92.276 72.924) (end 92.276 69.424) (width 0.8) (layer "B.Cu") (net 3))
 (segment (start 72.862 70.856) (end 72.862 73.4) (width 0.8) (layer "F.Cu") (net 7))
 (segment (start 105.524 59.362) (end 105.868 59.362) (width 0.4) (layer "F.Cu") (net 7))
 (segment (start 105.488 57.294) (end 105.524 57.33) (width 0.5) (layer "F.Cu") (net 7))
 (segment (start 109.3745 71.4255) (end 108.484 72.316) (width 0.6) (layer "F.Cu") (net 7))
 (segment (start 109.612 58.3685) (end 108.612 58.3685) (width 0.25) (layer "F.Cu") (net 7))
 (segment (start 72.862 75.876) (end 74.112 77.126) (width 0.8) (layer "F.Cu") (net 7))
 (segment (start 74.306 53.694) (end 70.08 57.92) (width 0.8) (layer "F.Cu") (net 7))
 (segment (start 106.812 70.325) (end 106.912 70.425) (width 0.25) (layer "F.Cu") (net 7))
 (segment (start 105.386 59.5) (end 105.524 59.362) (width 0.6) (layer "F.Cu") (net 7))
 (segment (start 108.484 72.316) (end 106.384 72.316) (width 0.6) (layer "F.Cu") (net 7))
 (segment (start 106.512 60.006) (end 107.1745 60.006) (width 0.4) (layer "F.Cu") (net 7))
 (segment (start 71 73.4) (end 72.862 73.4) (width 0.8) (layer "F.Cu") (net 7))
 (segment (start 105.524 57.224) (end 101.994 53.694) (width 0.8) (layer "F.Cu") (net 7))
 (segment (start 70.08 57.92) (end 70.08 72.48) (width 0.8) (layer "F.Cu") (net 7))
 (segment (start 74.112 77.126) (end 74.112 80.762) (width 0.8) (layer "F.Cu") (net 7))
 (segment (start 101.2 59.5) (end 105.386 59.5) (width 0.6) (layer "F.Cu") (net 7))
 (segment (start 105.524 57.33) (end 105.524 57.224) (width 0.8) (layer "F.Cu") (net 7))
 (segment (start 72.862 73.4) (end 72.862 75.876) (width 0.8) (layer "F.Cu") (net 7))
 (segment (start 107.394 60.006) (end 107.4 60) (width 0.4) (layer "F.Cu") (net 7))
 (segment (start 109.412 63.706) (end 109.412 65.9685) (width 0.4) (layer "F.Cu") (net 7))
 (segment (start 106.384 72.316) (end 105 73.7) (width 0.6) (layer "F.Cu") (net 7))
 (segment (start 105.524 57.33) (end 108.816 57.33) (width 0.4) (layer "F.Cu") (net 7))
 (segment (start 109.112 57.626) (end 109.112 58.3685) (width 0.4) (layer "F.Cu") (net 7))
 (segment (start 109.3745 66.006) (end 109.3745 71.4255) (width 0.6) (layer "F.Cu") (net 7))
 (segment (start 105 73.7) (end 99.2 73.7) (width 0.6) (layer "F.Cu") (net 7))
 (segment (start 105.868 59.362) (end 106.512 60.006) (width 0.4) (layer "F.Cu") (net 7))
 (segment (start 104.2 70.325) (end 106.812 70.325) (width 0.25) (layer "F.Cu") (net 7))
 (segment (start 109.612 62.2435) (end 109.612 63.506) (width 0.25) (layer "F.Cu") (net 7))
 (segment (start 98.6 62.1) (end 101.2 59.5) (width 0.6) (layer "F.Cu") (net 7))
 (segment (start 101.994 53.694) (end 74.306 53.694) (width 0.8) (layer "F.Cu") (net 7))
 (segment (start 109.612 63.506) (end 109.412 63.706) (width 0.4) (layer "F.Cu") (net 7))
 (segment (start 98.6 73.1) (end 98.6 62.1) (width 0.6) (layer "F.Cu") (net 7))
 (segment (start 74.112 80.762) (end 74.08 80.794) (width 0.8) (layer "F.Cu") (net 7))
 (segment (start 108.816 57.33) (end 109.112 57.626) (width 0.4) (layer "F.Cu") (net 7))
 (segment (start 99.2 73.7) (end 98.6 73.1) (width 0.6) (layer "F.Cu") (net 7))
 (segment (start 70.08 72.48) (end 71 73.4) (width 0.8) (layer "F.Cu") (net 7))
 (via (at 105.524 57.33) (size 1) (drill 0.4) (layers "F.Cu" "B.Cu") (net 7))
 (via (at 105.524 59.362) (size 1) (drill 0.4) (layers "F.Cu" "B.Cu") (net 7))
 (segment (start 105.524 57.33) (end 105.524 59.362) (width 0.25) (layer "B.Cu") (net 7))
 (segment (start 104.512 66.488) (end 104.512 64.206) (width 0.4) (layer "F.Cu") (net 10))
 (segment (start 104.2 66.8) (end 104.2 68.275) (width 0.4) (layer "F.Cu") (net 10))
 (segment (start 104.2 66.8) (end 104.512 66.488) (width 0.4) (layer "F.Cu") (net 10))
 (segment (start 106.912 68.606) (end 106.912 66.806) (width 0.4) (layer "F.Cu") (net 6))
 (segment (start 113.012 60.806) (end 113.712 60.106) (width 0.25) (layer "F.Cu") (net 13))
 (segment (start 111.0495 60.806) (end 113.012 60.806) (width 0.25) (layer "F.Cu") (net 13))
 (segment (start 112.312 60.206) (end 112.312 58.306) (width 0.25) (layer "F.Cu") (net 11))
 (segment (start 112.212 60.306) (end 112.312 60.206) (width 0.25) (layer "F.Cu") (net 11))
 (segment (start 111.0495 60.306) (end 112.212 60.306) (width 0.25) (layer "F.Cu") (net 11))
 (segment (start 112.812 57.806) (end 113.612 57.806) (width 0.25) (layer "F.Cu") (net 11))
 (segment (start 113.612 57.806) (end 113.712 57.706) (width 0.25) (layer "F.Cu") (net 11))
 (segment (start 112.312 58.306) (end 112.812 57.806) (width 0.25) (layer "F.Cu") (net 11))
 (segment (start 108.112 62.2435) (end 104.5495 62.2435) (width 0.25) (layer "F.Cu") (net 14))
 (segment (start 104.5495 62.2435) (end 104.512 62.206) (width 0.25) (layer "F.Cu") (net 14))
 (segment (start 108.612 62.2435) (end 108.612 63.206) (width 0.25) (layer "F.Cu") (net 5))
 (segment (start 108.612 63.206) (end 108.212 63.606) (width 0.25) (layer "F.Cu") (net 5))
 (segment (start 108.212 63.606) (end 107.312 63.606) (width 0.25) (layer "F.Cu") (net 5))
 (segment (start 106.912 64.006) (end 106.912 64.806) (width 0.25) (layer "F.Cu") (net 5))
 (segment (start 107.312 63.606) (end 106.912 64.006) (width 0.25) (layer "F.Cu") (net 5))
 (segment (start 103.362 61.056) (end 105.662 61.056) (width 0.25) (layer "F.Cu") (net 12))
 (segment (start 105.662 61.056) (end 105.912 61.306) (width 0.25) (layer "F.Cu") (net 12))
 (segment (start 103.28 77.894) (end 103.28 79.594) (width 0.4) (layer "F.Cu") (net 12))
 (segment (start 103.28 79.594) (end 103.88 80.194) (width 0.4) (layer "F.Cu") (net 12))
 (segment (start 102.4 72.1) (end 102.4 62.018) (width 0.25) (layer "F.Cu") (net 12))
 (segment (start 102.4 62.018) (end 103.362 61.056) (width 0.25) (layer "F.Cu") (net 12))
 (segment (start 105.912 61.306) (end 107.1745 61.306) (width 0.25) (layer "F.Cu") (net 12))
 (via (at 103.28 77.894) (size 1) (drill 0.4) (layers "F.Cu" "B.Cu") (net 12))
 (via (at 102.4 72.1) (size 1) (drill 0.4) (layers "F.Cu" "B.Cu") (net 12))
 (segment (start 102.476 77.09) (end 103.28 77.894) (width 0.4) (layer "B.Cu") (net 12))
 (segment (start 102.476 72.176) (end 102.476 77.09) (width 0.4) (layer "B.Cu") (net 12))
 (segment (start 102.4 72.1) (end 102.476 72.176) (width 0.4) (layer "B.Cu") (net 12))
 (segment (start 89.68 76.32) (end 89.68 79.894) (width 0.5) (layer "F.Cu") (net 9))
 (segment (start 86.4 73) (end 89.7 76.3) (width 0.5) (layer "F.Cu") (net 9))
 (segment (start 86.4 71.4) (end 86.4 69.2) (width 0.5) (layer "F.Cu") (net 9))
 (segment (start 86.4 69.2) (end 86.3 69.1) (width 0.5) (layer "F.Cu") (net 9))
 (segment (start 86.4 71.4) (end 86.4 73) (width 0.5) (layer "F.Cu") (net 9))
 (segment (start 89.7 76.3) (end 89.68 76.32) (width 0.5) (layer "F.Cu") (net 9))
 (segment (start 87.236 79.141) (end 87.18 79.197) (width 0.5) (layer "F.Cu") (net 8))
 (segment (start 76.1 69.4) (end 76.1 70.8) (width 0.5) (layer "F.Cu") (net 8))
 (segment (start 76.8 68.7) (end 76.1 69.4) (width 0.5) (layer "F.Cu") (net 8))
 (segment (start 81.8 74.6) (end 81.8 70.1) (width 0.5) (layer "F.Cu") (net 8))
 (segment (start 76.1 70.8) (end 74.918 70.8) (width 0.5) (layer "F.Cu") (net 8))
 (segment (start 87.18 79.197) (end 87.18 79.894) (width 0.5) (layer "F.Cu") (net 8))
 (segment (start 74.918 70.8) (end 74.862 70.856) (width 0.5) (layer "F.Cu") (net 8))
 (segment (start 87.18 79.894) (end 87.094 79.894) (width 0.5) (layer "F.Cu") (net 8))
 (segment (start 76.1 70.8) (end 77.206 70.8) (width 0.5) (layer "F.Cu") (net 8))
 (segment (start 87.094 79.894) (end 81.8 74.6) (width 0.5) (layer "F.Cu") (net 8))
 (segment (start 80.4 68.7) (end 76.8 68.7) (width 0.5) (layer "F.Cu") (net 8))
 (segment (start 81.8 70.1) (end 80.4 68.7) (width 0.5) (layer "F.Cu") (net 8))
 (segment (start 77.206 70.8) (end 77.262 70.856) (width 0.5) (layer "F.Cu") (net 8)))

